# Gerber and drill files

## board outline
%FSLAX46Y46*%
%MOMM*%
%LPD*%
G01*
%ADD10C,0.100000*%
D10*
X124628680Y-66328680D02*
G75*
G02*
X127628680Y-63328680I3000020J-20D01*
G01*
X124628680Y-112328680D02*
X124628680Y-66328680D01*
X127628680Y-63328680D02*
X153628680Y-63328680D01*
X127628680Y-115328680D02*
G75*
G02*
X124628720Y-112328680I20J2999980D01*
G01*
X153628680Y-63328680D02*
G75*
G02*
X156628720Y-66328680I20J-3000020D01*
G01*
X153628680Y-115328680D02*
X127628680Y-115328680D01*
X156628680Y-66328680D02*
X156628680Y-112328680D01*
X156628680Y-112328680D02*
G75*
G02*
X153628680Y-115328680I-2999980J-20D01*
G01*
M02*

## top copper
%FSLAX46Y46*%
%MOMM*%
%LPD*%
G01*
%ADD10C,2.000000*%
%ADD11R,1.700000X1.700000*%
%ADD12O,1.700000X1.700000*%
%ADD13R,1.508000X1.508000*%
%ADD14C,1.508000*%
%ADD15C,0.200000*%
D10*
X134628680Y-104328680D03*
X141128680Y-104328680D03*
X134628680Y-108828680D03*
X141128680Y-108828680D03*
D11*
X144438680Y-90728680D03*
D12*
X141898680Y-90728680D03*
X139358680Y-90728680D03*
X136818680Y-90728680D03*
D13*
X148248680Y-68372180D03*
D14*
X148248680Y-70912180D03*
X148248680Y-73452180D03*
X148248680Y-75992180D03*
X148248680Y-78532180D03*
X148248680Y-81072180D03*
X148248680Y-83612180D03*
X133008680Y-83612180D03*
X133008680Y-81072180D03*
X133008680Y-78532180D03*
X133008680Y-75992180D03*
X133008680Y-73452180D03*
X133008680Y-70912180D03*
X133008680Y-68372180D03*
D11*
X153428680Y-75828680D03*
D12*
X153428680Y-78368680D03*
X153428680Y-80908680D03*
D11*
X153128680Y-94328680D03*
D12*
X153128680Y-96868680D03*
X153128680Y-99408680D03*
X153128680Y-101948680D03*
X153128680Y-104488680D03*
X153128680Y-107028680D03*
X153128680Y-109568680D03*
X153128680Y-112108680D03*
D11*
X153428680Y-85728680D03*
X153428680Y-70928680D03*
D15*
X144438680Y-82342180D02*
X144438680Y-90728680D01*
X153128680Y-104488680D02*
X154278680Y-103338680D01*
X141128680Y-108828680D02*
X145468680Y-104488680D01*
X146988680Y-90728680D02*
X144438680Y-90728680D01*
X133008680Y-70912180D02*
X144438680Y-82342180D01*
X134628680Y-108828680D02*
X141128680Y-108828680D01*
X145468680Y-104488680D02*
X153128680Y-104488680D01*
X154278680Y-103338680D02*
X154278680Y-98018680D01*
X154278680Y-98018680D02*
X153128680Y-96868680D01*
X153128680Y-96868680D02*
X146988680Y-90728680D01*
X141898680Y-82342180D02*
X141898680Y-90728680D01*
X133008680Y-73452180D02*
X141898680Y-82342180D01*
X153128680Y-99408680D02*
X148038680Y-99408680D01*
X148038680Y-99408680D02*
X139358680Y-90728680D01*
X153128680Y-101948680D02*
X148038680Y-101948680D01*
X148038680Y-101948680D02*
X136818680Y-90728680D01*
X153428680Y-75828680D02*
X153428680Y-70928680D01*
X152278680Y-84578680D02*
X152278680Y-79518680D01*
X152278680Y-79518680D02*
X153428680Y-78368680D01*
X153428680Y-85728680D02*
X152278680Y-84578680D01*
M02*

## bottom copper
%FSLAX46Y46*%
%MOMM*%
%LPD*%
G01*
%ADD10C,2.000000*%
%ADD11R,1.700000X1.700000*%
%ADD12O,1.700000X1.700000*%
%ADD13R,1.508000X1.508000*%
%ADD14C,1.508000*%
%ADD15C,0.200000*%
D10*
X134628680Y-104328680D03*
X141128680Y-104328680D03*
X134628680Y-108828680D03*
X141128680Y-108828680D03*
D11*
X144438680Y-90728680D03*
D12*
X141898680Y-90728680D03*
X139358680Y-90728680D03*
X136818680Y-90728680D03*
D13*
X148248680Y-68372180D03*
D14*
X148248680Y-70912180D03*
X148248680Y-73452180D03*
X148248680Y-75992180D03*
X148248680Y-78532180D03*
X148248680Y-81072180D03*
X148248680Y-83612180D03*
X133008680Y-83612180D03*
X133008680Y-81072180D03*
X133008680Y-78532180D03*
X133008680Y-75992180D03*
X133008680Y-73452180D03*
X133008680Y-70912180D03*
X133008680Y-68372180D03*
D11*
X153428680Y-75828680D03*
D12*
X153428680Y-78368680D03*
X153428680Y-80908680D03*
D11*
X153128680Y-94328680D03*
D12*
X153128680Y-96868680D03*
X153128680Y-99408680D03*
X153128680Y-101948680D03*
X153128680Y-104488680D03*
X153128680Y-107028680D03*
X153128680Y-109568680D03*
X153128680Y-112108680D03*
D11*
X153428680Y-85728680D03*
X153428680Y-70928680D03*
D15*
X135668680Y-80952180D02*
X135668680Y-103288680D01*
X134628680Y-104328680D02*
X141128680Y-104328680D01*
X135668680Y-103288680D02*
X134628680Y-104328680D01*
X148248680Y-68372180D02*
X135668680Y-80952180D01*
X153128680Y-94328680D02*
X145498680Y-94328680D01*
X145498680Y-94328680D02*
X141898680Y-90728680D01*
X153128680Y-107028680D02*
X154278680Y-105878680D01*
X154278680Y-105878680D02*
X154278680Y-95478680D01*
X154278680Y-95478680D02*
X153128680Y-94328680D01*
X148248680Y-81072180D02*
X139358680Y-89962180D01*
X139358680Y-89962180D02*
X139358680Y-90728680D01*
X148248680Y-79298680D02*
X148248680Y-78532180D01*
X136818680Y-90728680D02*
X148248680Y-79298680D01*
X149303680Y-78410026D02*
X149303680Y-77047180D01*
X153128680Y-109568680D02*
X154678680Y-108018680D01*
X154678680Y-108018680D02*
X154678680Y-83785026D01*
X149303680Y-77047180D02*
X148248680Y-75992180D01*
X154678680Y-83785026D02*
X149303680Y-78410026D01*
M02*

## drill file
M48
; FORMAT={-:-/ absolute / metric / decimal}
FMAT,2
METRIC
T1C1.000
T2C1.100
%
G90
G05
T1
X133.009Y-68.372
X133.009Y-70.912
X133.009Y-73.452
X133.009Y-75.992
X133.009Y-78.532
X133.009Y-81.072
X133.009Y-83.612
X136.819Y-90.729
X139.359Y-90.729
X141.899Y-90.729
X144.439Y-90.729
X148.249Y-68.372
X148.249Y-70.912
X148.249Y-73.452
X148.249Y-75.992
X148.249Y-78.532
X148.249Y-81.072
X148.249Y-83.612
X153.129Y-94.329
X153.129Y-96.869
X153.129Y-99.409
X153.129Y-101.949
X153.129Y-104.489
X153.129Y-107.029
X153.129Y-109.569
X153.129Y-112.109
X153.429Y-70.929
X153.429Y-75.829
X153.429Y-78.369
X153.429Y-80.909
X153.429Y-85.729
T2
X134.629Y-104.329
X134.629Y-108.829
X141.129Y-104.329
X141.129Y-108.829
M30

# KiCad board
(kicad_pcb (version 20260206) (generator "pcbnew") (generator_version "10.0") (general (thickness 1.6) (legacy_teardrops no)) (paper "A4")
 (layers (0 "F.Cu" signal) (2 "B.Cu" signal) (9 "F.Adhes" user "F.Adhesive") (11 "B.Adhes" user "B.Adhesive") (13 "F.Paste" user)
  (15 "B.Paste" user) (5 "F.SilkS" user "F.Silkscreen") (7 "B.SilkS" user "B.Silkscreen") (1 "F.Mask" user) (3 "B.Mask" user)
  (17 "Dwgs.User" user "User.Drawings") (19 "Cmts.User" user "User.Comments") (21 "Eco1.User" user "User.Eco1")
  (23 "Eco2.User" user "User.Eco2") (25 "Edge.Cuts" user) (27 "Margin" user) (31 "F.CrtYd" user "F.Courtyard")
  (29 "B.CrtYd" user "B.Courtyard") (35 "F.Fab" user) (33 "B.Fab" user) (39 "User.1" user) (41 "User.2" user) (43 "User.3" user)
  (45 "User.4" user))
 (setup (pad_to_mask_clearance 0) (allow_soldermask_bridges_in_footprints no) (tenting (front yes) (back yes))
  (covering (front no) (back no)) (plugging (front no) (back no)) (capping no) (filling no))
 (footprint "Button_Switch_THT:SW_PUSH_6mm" (layer "F.Cu") (at 134.62868 104.32868)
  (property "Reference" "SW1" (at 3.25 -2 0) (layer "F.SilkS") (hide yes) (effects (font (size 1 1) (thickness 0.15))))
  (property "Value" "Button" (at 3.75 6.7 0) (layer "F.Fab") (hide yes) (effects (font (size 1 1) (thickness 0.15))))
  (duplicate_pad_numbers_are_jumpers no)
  (pad "1" thru_hole circle (at 0 0 90) (size 2 2) (drill 1.1) (layers "*.Cu" "*.Mask") (remove_unused_layers no) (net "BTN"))
  (pad "1" thru_hole circle (at 6.5 0 90) (size 2 2) (drill 1.1) (layers "*.Cu" "*.Mask") (remove_unused_layers no) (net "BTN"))
  (pad "2" thru_hole circle (at 0 4.5 90) (size 2 2) (drill 1.1) (layers "*.Cu" "*.Mask") (remove_unused_layers no) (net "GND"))
  (pad "2" thru_hole circle (at 6.5 4.5 90) (size 2 2) (drill 1.1) (layers "*.Cu" "*.Mask") (remove_unused_layers no) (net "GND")))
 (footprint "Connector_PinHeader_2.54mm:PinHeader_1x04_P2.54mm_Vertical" (layer "F.Cu") (at 144.43868 90.72868 -90)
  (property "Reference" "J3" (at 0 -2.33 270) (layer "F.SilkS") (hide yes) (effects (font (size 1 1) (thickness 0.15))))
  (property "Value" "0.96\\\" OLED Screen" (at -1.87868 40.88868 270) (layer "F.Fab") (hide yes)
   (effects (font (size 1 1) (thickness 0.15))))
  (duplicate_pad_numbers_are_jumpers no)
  (pad "1" thru_hole rect (at 0 0 270) (size 1.7 1.7) (drill 1) (layers "*.Cu" "*.Mask") (remove_unused_layers no) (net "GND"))
  (pad "2" thru_hole oval (at 0 2.54 270) (size 1.7 1.7) (drill 1) (layers "*.Cu" "*.Mask") (remove_unused_layers no) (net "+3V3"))
  (pad "3" thru_hole oval (at 0 5.08 270) (size 1.7 1.7) (drill 1) (layers "*.Cu" "*.Mask") (remove_unused_layers no) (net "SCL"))
  (pad "4" thru_hole oval (at 0 7.62 270) (size 1.7 1.7) (drill 1) (layers "*.Cu" "*.Mask") (remove_unused_layers no) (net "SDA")))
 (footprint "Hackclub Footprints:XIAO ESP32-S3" (layer "B.Cu") (at 140.62868 75.92868 180)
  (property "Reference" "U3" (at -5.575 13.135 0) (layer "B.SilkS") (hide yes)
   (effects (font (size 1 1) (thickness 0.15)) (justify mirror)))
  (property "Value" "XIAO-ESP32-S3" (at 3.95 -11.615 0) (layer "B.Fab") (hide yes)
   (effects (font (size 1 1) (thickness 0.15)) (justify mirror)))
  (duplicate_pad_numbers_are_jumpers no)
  (pad "1" thru_hole rect (at -7.62 7.5565 180) (size 1.508 1.508) (drill 1) (layers "*.Cu" "*.Mask") (remove_unused_layers no) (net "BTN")
   (solder_mask_margin 0.102))
  (pad "2" thru_hole circle (at -7.62 5.0165 180) (size 1.508 1.508) (drill 1) (layers "*.Cu" "*.Mask") (remove_unused_layers no)
   (solder_mask_margin 0.102))
  (pad "3" thru_hole circle (at -7.62 2.4765 180) (size 1.508 1.508) (drill 1) (layers "*.Cu" "*.Mask") (remove_unused_layers no)
   (solder_mask_margin 0.102))
  (pad "4" thru_hole circle (at -7.62 -0.0635 180) (size 1.508 1.508) (drill 1) (layers "*.Cu" "*.Mask") (remove_unused_layers no)
   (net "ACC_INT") (solder_mask_margin 0.102))
  (pad "5" thru_hole circle (at -7.62 -2.6035 180) (size 1.508 1.508) (drill 1) (layers "*.Cu" "*.Mask") (remove_unused_layers no)
   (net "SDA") (solder_mask_margin 0.102))
  (pad "6" thru_hole circle (at -7.62 -5.1435 180) (size 1.508 1.508) (drill 1) (layers "*.Cu" "*.Mask") (remove_unused_layers no)
   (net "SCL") (solder_mask_margin 0.102))
  (pad "7" thru_hole circle (at -7.62 -7.6835 180) (size 1.508 1.508) (drill 1) (layers "*.Cu" "*.Mask") (remove_unused_layers no)
   (solder_mask_margin 0.102))
  (pad "8" thru_hole circle (at 7.62 -7.6835 180) (size 1.508 1.508) (drill 1) (layers "*.Cu" "*.Mask") (remove_unused_layers no)
   (solder_mask_margin 0.102))
  (pad "9" thru_hole circle (at 7.62 -5.1435 180) (size 1.508 1.508) (drill 1) (layers "*.Cu" "*.Mask") (remove_unused_layers no)
   (solder_mask_margin 0.102))
  (pad "10" thru_hole circle (at 7.62 -2.6035 180) (size 1.508 1.508) (drill 1) (layers "*.Cu" "*.Mask") (remove_unused_layers no)
   (solder_mask_margin 0.102))
  (pad "11" thru_hole circle (at 7.62 -0.0635 180) (size 1.508 1.508) (drill 1) (layers "*.Cu" "*.Mask") (remove_unused_layers no)
   (solder_mask_margin 0.102))
  (pad "12" thru_hole circle (at 7.62 2.4765 180) (size 1.508 1.508) (drill 1) (layers "*.Cu" "*.Mask") (remove_unused_layers no)
   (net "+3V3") (solder_mask_margin 0.102))
  (pad "13" thru_hole circle (at 7.62 5.0165 180) (size 1.508 1.508) (drill 1) (layers "*.Cu" "*.Mask") (remove_unused_layers no)
   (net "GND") (solder_mask_margin 0.102))
  (pad "14" thru_hole circle (at 7.62 7.5565 180) (size 1.508 1.508) (drill 1) (layers "*.Cu" "*.Mask") (remove_unused_layers no)
   (solder_mask_margin 0.102)))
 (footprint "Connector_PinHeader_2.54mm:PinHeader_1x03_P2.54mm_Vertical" (layer "B.Cu") (at 153.42868 75.82868 180)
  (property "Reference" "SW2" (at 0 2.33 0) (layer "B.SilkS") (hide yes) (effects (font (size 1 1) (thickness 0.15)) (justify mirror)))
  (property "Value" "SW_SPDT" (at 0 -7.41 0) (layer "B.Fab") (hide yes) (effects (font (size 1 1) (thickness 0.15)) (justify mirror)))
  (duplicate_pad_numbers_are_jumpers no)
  (pad "1" thru_hole rect (at 0 0 180) (size 1.7 1.7) (drill 1) (layers "*.Cu" "*.Mask") (remove_unused_layers no) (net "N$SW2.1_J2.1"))
  (pad "2" thru_hole oval (at 0 -2.54 180) (size 1.7 1.7) (drill 1) (layers "*.Cu" "*.Mask") (remove_unused_layers no) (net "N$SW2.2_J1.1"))
  (pad "3" thru_hole oval (at 0 -5.08 180) (size 1.7 1.7) (drill 1) (layers "*.Cu" "*.Mask") (remove_unused_layers no)))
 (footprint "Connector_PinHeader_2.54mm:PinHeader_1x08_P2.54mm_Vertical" (layer "B.Cu") (at 153.12868 94.32868 180)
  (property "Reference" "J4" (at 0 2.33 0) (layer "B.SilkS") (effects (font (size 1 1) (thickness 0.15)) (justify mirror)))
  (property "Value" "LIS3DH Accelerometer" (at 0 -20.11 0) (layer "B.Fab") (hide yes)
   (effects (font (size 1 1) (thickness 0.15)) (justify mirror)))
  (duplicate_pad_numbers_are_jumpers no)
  (pad "1" thru_hole rect (at 0 0 180) (size 1.7 1.7) (drill 1) (layers "*.Cu" "*.Mask") (remove_unused_layers no) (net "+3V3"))
  (pad "2" thru_hole oval (at 0 -2.54 180) (size 1.7 1.7) (drill 1) (layers "*.Cu" "*.Mask") (remove_unused_layers no) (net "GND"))
  (pad "3" thru_hole oval (at 0 -5.08 180) (size 1.7 1.7) (drill 1) (layers "*.Cu" "*.Mask") (remove_unused_layers no) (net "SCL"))
  (pad "4" thru_hole oval (at 0 -7.62 180) (size 1.7 1.7) (drill 1) (layers "*.Cu" "*.Mask") (remove_unused_layers no) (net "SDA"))
  (pad "5" thru_hole oval (at 0 -10.16 180) (size 1.7 1.7) (drill 1) (layers "*.Cu" "*.Mask") (remove_unused_layers no) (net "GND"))
  (pad "6" thru_hole oval (at 0 -12.7 180) (size 1.7 1.7) (drill 1) (layers "*.Cu" "*.Mask") (remove_unused_layers no) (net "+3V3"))
  (pad "7" thru_hole oval (at 0 -15.24 180) (size 1.7 1.7) (drill 1) (layers "*.Cu" "*.Mask") (remove_unused_layers no) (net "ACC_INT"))
  (pad "8" thru_hole oval (at 0 -17.78 180) (size 1.7 1.7) (drill 1) (layers "*.Cu" "*.Mask") (remove_unused_layers no)))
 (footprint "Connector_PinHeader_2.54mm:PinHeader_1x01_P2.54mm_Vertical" (layer "B.Cu") (at 153.42868 85.72868 180)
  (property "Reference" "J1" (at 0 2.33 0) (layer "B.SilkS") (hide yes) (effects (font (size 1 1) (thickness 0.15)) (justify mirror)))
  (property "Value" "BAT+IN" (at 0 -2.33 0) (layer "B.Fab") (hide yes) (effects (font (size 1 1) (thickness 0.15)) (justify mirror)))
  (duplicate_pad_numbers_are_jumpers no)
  (pad "1" thru_hole rect (at 0 0 180) (size 1.7 1.7) (drill 1) (layers "*.Cu" "*.Mask") (remove_unused_layers no) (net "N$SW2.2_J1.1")))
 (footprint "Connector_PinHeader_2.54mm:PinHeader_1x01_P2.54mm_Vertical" (layer "B.Cu") (at 153.42868 70.92868 180)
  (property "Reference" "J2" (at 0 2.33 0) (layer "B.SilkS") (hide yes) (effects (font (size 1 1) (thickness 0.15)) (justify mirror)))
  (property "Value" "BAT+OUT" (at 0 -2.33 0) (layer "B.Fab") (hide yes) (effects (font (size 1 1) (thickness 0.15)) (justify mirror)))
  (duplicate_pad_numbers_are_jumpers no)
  (pad "1" thru_hole rect (at 0 0 180) (size 1.7 1.7) (drill 1) (layers "*.Cu" "*.Mask") (remove_unused_layers no) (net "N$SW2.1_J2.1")))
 (gr_arc (start 124.62868 66.32868) (mid 125.50736 64.20736) (end 127.62868 63.32868) (stroke (width 0.1) (type default))
  (layer "Edge.Cuts"))
 (gr_line (start 124.62868 112.32868) (end 124.62868 66.32868) (stroke (width 0.1) (type default)) (layer "Edge.Cuts"))
 (gr_line (start 127.62868 63.32868) (end 153.62868 63.32868) (stroke (width 0.1) (type default)) (layer "Edge.Cuts"))
 (gr_arc (start 127.62868 115.32868) (mid 125.50736 114.45) (end 124.62868 112.32868) (stroke (width 0.1) (type default))
  (layer "Edge.Cuts"))
 (gr_arc (start 153.62868 63.32868) (mid 155.75 64.20736) (end 156.62868 66.32868) (stroke (width 0.1) (type default)) (layer "Edge.Cuts"))
 (gr_line (start 153.62868 115.32868) (end 127.62868 115.32868) (stroke (width 0.1) (type default)) (layer "Edge.Cuts"))
 (gr_line (start 156.62868 66.32868) (end 156.62868 112.32868) (stroke (width 0.1) (type default)) (layer "Edge.Cuts"))
 (gr_arc (start 156.62868 112.32868) (mid 155.75 114.45) (end 153.62868 115.32868) (stroke (width 0.1) (type default)) (layer "Edge.Cuts"))
 (segment (start 135.66868 80.95218) (end 135.66868 103.28868) (width 0.2) (layer "B.Cu") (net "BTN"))
 (segment (start 134.62868 104.32868) (end 141.12868 104.32868) (width 0.2) (layer "B.Cu") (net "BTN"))
 (segment (start 135.66868 103.28868) (end 134.62868 104.32868) (width 0.2) (layer "B.Cu") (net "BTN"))
 (segment (start 148.24868 68.37218) (end 135.66868 80.95218) (width 0.2) (layer "B.Cu") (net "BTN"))
 (segment (start 144.43868 82.34218) (end 144.43868 90.72868) (width 0.2) (layer "F.Cu") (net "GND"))
 (segment (start 153.12868 104.48868) (end 154.27868 103.33868) (width 0.2) (layer "F.Cu") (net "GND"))
 (segment (start 141.12868 108.82868) (end 145.46868 104.48868) (width 0.2) (layer "F.Cu") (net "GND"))
 (segment (start 146.98868 90.72868) (end 144.43868 90.72868) (width 0.2) (layer "F.Cu") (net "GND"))
 (segment (start 133.00868 70.91218) (end 144.43868 82.34218) (width 0.2) (layer "F.Cu") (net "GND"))
 (segment (start 134.62868 108.82868) (end 141.12868 108.82868) (width 0.2) (layer "F.Cu") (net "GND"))
 (segment (start 145.46868 104.48868) (end 153.12868 104.48868) (width 0.2) (layer "F.Cu") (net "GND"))
 (segment (start 154.27868 103.33868) (end 154.27868 98.01868) (width 0.2) (layer "F.Cu") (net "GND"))
 (segment (start 154.27868 98.01868) (end 153.12868 96.86868) (width 0.2) (layer "F.Cu") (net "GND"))
 (segment (start 153.12868 96.86868) (end 146.98868 90.72868) (width 0.2) (layer "F.Cu") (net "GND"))
 (segment (start 141.89868 82.34218) (end 141.89868 90.72868) (width 0.2) (layer "F.Cu") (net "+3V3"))
 (segment (start 133.00868 73.45218) (end 141.89868 82.34218) (width 0.2) (layer "F.Cu") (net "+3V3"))
 (segment (start 153.12868 94.32868) (end 145.49868 94.32868) (width 0.2) (layer "B.Cu") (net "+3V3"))
 (segment (start 145.49868 94.32868) (end 141.89868 90.72868) (width 0.2) (layer "B.Cu") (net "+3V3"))
 (segment (start 153.12868 107.02868) (end 154.27868 105.87868) (width 0.2) (layer "B.Cu") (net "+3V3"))
 (segment (start 154.27868 105.87868) (end 154.27868 95.47868) (width 0.2) (layer "B.Cu") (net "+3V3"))
 (segment (start 154.27868 95.47868) (end 153.12868 94.32868) (width 0.2) (layer "B.Cu") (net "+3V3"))
 (segment (start 153.12868 99.40868) (end 148.03868 99.40868) (width 0.2) (layer "F.Cu") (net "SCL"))
 (segment (start 148.03868 99.40868) (end 139.35868 90.72868) (width 0.2) (layer "F.Cu") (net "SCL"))
 (segment (start 148.24868 81.07218) (end 139.35868 89.96218) (width 0.2) (layer "B.Cu") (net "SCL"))
 (segment (start 139.35868 89.96218) (end 139.35868 90.72868) (width 0.2) (layer "B.Cu") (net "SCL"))
 (segment (start 153.12868 101.94868) (end 148.03868 101.94868) (width 0.2) (layer "F.Cu") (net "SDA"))
 (segment (start 148.03868 101.94868) (end 136.81868 90.72868) (width 0.2) (layer "F.Cu") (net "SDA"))
 (segment (start 148.24868 79.29868) (end 148.24868 78.53218) (width 0.2) (layer "B.Cu") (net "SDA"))
 (segment (start 136.81868 90.72868) (end 148.24868 79.29868) (width 0.2) (layer "B.Cu") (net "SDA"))
 (segment (start 149.30368 78.410026) (end 149.30368 77.04718) (width 0.2) (layer "B.Cu") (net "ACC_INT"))
 (segment (start 153.12868 109.56868) (end 154.67868 108.01868) (width 0.2) (layer "B.Cu") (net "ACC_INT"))
 (segment (start 154.67868 108.01868) (end 154.67868 83.785026) (width 0.2) (layer "B.Cu") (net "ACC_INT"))
 (segment (start 149.30368 77.04718) (end 148.24868 75.99218) (width 0.2) (layer "B.Cu") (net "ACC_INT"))
 (segment (start 154.67868 83.785026) (end 149.30368 78.410026) (width 0.2) (layer "B.Cu") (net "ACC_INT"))
 (segment (start 153.42868 75.82868) (end 153.42868 70.92868) (width 0.2) (layer "F.Cu") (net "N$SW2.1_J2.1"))
 (segment (start 152.27868 84.57868) (end 152.27868 79.51868) (width 0.2) (layer "F.Cu") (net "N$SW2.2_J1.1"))
 (segment (start 152.27868 79.51868) (end 153.42868 78.36868) (width 0.2) (layer "F.Cu") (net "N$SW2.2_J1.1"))
 (segment (start 153.42868 85.72868) (end 152.27868 84.57868) (width 0.2) (layer "F.Cu") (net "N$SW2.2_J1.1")))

